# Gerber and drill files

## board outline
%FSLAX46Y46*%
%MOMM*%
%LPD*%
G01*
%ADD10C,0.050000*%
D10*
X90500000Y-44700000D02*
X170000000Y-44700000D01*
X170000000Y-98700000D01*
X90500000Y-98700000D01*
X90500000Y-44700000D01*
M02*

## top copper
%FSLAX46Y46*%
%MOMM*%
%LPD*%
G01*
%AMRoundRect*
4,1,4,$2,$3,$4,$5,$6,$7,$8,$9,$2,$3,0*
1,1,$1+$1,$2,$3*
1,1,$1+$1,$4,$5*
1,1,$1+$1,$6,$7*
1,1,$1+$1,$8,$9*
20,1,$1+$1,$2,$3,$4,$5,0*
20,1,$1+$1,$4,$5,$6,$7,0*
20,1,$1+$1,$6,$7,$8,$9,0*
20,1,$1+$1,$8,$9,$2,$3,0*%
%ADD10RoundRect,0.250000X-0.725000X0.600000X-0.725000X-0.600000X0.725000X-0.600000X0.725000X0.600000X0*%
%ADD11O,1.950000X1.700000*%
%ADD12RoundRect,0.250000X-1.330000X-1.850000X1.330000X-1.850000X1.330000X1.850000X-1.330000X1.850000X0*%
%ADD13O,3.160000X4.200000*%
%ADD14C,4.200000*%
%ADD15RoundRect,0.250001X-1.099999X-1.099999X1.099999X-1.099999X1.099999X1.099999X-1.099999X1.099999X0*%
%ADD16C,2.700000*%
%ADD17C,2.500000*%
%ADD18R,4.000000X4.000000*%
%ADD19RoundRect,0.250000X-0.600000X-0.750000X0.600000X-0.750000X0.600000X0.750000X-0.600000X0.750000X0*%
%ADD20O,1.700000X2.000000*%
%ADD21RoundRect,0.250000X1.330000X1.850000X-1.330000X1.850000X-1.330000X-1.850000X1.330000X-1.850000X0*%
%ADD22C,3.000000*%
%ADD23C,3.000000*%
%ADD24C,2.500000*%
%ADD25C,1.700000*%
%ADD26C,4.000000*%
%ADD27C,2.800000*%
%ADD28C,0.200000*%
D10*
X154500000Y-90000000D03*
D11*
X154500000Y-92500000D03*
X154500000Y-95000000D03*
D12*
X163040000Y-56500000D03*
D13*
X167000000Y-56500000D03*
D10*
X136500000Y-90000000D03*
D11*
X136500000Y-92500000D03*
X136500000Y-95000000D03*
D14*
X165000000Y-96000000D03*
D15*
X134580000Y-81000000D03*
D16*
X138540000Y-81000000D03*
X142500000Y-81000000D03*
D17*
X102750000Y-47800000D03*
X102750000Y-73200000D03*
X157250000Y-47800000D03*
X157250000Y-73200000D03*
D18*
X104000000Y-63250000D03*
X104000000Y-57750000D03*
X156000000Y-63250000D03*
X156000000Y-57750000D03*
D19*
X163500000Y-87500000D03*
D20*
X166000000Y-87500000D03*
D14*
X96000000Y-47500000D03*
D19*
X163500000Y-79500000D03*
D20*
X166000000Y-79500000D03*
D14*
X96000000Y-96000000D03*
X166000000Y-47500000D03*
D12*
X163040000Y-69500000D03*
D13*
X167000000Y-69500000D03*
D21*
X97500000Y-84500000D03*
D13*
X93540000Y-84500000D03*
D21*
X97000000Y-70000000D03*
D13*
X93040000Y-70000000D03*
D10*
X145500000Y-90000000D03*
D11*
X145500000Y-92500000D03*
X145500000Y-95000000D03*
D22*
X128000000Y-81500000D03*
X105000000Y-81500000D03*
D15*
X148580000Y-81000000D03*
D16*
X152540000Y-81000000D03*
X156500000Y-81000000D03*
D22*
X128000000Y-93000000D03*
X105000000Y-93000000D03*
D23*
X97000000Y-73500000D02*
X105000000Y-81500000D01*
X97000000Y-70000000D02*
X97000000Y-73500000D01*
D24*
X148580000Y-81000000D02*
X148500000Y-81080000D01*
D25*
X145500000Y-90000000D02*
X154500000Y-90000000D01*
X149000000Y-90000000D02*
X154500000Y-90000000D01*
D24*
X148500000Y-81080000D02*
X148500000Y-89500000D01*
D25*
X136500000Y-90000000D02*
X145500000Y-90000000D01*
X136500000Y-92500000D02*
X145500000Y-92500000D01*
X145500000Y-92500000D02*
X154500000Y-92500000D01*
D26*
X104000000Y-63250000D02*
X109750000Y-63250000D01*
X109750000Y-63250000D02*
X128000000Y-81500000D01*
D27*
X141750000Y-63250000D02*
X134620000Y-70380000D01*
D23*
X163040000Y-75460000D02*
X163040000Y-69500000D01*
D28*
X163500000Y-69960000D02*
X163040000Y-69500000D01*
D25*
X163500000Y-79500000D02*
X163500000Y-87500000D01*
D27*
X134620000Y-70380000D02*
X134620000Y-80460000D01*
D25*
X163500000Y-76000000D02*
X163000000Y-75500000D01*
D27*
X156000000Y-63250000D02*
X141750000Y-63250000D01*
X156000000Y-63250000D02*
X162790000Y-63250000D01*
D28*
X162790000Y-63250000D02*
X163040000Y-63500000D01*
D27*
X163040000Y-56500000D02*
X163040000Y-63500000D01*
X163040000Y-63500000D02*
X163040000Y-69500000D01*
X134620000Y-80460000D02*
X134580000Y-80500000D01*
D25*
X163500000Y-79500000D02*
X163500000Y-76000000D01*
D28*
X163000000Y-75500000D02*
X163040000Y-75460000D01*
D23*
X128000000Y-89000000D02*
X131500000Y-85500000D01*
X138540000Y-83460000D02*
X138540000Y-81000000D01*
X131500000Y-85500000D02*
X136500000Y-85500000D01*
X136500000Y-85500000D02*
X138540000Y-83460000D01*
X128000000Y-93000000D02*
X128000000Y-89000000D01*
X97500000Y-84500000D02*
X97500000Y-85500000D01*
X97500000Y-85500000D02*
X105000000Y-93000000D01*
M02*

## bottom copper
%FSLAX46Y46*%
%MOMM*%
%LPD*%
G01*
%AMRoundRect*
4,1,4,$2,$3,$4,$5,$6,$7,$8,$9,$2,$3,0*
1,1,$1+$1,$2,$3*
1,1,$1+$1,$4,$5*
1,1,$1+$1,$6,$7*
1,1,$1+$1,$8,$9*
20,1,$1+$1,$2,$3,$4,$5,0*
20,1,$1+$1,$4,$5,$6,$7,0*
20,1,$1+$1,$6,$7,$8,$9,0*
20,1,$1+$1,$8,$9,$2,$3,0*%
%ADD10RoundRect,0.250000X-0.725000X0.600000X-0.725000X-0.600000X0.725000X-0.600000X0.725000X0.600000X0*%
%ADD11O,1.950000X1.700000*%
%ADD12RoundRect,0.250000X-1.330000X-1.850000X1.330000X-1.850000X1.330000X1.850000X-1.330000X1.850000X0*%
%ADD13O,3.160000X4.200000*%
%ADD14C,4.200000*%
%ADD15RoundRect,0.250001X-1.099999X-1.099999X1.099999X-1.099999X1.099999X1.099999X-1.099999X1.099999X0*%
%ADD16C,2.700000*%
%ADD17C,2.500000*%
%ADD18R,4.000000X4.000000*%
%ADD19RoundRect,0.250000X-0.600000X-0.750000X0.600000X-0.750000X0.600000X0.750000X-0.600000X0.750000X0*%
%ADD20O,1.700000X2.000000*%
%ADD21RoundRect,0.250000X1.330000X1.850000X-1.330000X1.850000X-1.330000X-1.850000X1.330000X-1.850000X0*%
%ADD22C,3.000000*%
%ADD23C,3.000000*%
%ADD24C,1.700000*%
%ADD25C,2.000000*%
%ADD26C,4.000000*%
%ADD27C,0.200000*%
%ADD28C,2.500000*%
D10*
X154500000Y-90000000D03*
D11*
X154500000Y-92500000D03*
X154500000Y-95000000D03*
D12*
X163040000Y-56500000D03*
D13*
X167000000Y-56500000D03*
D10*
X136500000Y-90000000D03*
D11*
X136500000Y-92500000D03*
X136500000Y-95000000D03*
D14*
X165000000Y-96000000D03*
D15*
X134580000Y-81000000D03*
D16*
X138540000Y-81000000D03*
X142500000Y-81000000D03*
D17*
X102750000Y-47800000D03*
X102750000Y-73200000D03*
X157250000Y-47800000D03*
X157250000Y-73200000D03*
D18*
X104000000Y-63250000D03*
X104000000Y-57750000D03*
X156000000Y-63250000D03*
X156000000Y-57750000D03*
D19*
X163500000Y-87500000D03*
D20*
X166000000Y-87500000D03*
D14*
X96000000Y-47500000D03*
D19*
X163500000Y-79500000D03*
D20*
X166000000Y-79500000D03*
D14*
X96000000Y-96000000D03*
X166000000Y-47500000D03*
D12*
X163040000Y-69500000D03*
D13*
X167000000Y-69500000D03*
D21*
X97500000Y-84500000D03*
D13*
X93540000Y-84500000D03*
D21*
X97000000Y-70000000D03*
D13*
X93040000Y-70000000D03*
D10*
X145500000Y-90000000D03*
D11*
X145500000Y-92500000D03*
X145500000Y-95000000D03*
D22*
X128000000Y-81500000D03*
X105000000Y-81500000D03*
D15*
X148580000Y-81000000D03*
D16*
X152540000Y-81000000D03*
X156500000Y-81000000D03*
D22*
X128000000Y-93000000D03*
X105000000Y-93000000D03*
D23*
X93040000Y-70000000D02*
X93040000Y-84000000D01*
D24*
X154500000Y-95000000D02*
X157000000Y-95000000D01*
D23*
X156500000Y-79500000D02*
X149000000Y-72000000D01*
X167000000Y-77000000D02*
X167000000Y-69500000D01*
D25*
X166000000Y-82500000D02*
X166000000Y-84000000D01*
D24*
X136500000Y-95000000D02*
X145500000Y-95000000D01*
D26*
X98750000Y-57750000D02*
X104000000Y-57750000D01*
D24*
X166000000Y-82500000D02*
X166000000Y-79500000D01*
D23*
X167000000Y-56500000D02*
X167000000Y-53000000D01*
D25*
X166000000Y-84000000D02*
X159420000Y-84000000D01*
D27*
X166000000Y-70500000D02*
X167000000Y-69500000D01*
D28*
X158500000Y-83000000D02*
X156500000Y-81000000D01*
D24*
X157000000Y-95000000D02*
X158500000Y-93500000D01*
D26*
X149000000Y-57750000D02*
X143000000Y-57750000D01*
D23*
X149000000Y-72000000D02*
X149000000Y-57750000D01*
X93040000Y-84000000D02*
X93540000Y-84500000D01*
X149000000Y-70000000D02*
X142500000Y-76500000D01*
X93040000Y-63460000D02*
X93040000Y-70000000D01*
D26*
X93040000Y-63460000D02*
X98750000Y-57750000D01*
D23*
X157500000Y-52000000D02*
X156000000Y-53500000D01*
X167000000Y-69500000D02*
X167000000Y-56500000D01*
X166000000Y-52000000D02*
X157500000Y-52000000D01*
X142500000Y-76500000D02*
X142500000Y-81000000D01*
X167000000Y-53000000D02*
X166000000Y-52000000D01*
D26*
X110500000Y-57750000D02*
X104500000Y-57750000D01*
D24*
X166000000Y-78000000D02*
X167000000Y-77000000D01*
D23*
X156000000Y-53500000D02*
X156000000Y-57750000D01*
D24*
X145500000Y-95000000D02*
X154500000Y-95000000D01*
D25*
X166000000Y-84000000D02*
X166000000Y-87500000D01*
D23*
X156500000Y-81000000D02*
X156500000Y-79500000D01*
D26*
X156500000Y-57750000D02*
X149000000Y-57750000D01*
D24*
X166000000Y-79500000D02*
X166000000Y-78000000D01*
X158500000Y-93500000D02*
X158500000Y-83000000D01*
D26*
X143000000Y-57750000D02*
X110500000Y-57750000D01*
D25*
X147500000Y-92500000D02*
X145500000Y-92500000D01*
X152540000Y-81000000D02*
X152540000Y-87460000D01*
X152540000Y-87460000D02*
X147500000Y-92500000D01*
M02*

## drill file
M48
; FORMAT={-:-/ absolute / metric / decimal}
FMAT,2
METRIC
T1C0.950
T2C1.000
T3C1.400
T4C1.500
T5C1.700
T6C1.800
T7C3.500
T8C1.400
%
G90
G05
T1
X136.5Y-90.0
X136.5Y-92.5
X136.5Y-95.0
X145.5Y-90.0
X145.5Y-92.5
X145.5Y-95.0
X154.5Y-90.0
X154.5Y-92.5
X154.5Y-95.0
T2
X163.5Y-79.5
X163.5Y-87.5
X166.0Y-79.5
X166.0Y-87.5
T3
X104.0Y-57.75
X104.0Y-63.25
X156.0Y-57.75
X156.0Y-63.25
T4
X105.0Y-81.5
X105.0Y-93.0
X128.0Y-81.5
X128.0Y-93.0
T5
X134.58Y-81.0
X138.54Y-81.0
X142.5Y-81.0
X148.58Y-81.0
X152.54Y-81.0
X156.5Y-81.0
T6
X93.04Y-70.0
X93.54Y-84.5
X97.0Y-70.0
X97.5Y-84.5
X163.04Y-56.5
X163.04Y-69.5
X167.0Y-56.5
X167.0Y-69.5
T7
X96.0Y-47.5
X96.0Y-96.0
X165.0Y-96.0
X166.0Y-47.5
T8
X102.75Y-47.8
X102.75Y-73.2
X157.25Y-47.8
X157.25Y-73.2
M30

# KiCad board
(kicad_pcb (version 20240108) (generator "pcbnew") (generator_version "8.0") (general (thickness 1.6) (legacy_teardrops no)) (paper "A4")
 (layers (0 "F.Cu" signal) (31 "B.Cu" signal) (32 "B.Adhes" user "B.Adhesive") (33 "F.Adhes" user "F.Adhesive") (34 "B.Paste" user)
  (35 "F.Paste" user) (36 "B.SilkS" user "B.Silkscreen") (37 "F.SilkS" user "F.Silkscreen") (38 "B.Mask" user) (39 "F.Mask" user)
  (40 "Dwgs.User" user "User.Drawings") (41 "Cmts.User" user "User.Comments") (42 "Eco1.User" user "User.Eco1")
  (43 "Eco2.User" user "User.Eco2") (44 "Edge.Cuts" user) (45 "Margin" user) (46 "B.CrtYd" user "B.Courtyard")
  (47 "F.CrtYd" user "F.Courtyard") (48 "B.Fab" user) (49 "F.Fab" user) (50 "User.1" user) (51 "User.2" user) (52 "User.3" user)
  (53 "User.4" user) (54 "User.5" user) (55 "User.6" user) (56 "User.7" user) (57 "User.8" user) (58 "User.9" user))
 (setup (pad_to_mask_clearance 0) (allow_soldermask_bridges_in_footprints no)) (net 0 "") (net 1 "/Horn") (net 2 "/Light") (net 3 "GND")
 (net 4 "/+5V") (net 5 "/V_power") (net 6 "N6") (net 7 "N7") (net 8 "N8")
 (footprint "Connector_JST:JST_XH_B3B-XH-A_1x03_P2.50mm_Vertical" (layer "F.Cu") (at 154.5 90 -90)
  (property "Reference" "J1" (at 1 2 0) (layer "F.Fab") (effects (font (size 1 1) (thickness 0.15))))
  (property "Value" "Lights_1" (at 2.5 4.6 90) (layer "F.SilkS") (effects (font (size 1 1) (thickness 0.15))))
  (pad "1" thru_hole roundrect (at 0 0 270) (size 1.7 1.95) (drill 0.95) (layers "*.Cu" "*.Mask") (remove_unused_layers no)
   (roundrect_rratio 0.147059) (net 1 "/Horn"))
  (pad "2" thru_hole oval (at 2.5 0 270) (size 1.7 1.95) (drill 0.95) (layers "*.Cu" "*.Mask") (remove_unused_layers no) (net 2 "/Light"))
  (pad "3" thru_hole oval (at 5 0 270) (size 1.7 1.95) (drill 0.95) (layers "*.Cu" "*.Mask") (remove_unused_layers no) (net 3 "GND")))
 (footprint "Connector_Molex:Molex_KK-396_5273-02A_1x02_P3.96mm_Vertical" (layer "F.Cu") (at 163.04 56.5)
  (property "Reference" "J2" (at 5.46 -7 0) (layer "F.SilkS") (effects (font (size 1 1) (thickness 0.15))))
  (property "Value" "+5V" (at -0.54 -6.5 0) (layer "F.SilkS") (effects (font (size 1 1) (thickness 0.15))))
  (pad "1" thru_hole roundrect (at 0 0) (size 3.16 4.2) (drill 1.8) (layers "*.Cu" "*.Mask") (remove_unused_layers no)
   (roundrect_rratio 0.079114) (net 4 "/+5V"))
  (pad "2" thru_hole oval (at 3.96 0) (size 3.16 4.2) (drill 1.8) (layers "*.Cu" "*.Mask") (remove_unused_layers no) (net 3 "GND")))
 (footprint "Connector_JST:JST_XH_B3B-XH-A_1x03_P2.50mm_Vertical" (layer "F.Cu") (at 136.5 90 -90)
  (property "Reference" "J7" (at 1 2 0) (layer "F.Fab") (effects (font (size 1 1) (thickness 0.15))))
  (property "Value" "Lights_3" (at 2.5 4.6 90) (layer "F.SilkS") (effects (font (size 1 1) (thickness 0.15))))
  (pad "1" thru_hole roundrect (at 0 0 270) (size 1.7 1.95) (drill 0.95) (layers "*.Cu" "*.Mask") (remove_unused_layers no)
   (roundrect_rratio 0.147059) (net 1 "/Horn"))
  (pad "2" thru_hole oval (at 2.5 0 270) (size 1.7 1.95) (drill 0.95) (layers "*.Cu" "*.Mask") (remove_unused_layers no) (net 2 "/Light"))
  (pad "3" thru_hole oval (at 5 0 270) (size 1.7 1.95) (drill 0.95) (layers "*.Cu" "*.Mask") (remove_unused_layers no) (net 3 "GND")))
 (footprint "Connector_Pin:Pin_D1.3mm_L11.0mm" (layer "F.Cu") (at 165 96)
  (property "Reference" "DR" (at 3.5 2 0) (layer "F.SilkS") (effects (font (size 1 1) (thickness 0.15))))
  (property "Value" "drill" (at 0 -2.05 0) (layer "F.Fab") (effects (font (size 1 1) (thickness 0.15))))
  (pad "1" thru_hole circle (at 0 0) (size 4.2 4.2) (drill 3.5) (layers "*.Cu" "*.Mask") (remove_unused_layers no)))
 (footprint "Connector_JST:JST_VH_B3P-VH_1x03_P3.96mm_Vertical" (layer "F.Cu") (at 134.58 81)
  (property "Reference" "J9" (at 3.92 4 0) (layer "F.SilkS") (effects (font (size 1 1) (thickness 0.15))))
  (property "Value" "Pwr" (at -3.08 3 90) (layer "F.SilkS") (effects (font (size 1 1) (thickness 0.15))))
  (pad "1" thru_hole roundrect (at 0 0) (size 2.7 2.7) (drill 1.7) (layers "*.Cu" "*.Mask") (remove_unused_layers no)
   (roundrect_rratio 0.092593) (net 4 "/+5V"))
  (pad "2" thru_hole circle (at 3.96 0) (size 2.7 2.7) (drill 1.7) (layers "*.Cu" "*.Mask") (remove_unused_layers no) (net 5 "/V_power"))
  (pad "3" thru_hole circle (at 7.92 0) (size 2.7 2.7) (drill 1.7) (layers "*.Cu" "*.Mask") (remove_unused_layers no) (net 3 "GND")))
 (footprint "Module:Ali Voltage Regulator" (layer "F.Cu") (at 100 45.5)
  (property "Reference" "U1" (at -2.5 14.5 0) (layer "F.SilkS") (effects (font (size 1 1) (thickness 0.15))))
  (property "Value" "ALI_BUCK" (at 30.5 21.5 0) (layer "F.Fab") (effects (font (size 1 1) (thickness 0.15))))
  (pad "" np_thru_hole circle (at 2.75 2.3) (size 2.5 2.5) (drill 1.4) (layers "*.Cu" "*.Mask") (thermal_bridge_angle 90))
  (pad "" np_thru_hole circle (at 2.75 27.7) (size 2.5 2.5) (drill 1.4) (layers "*.Cu" "*.Mask"))
  (pad "" np_thru_hole circle (at 57.25 2.3) (size 2.5 2.5) (drill 1.4) (layers "*.Cu" "*.Mask"))
  (pad "" np_thru_hole circle (at 57.25 27.7) (size 2.5 2.5) (drill 1.4) (layers "*.Cu" "*.Mask"))
  (pad "1" thru_hole rect (at 4 17.75) (size 4 4) (drill 1.4) (layers "*.Cu" "*.Mask") (remove_unused_layers no) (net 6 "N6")
   (thermal_bridge_angle 45))
  (pad "2" thru_hole rect (at 4 12.25) (size 4 4) (drill 1.4) (layers "*.Cu" "*.Mask") (remove_unused_layers no) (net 3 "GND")
   (thermal_bridge_angle 45))
  (pad "3" thru_hole rect (at 56 17.75) (size 4 4) (drill 1.4) (layers "*.Cu" "*.Mask") (remove_unused_layers no) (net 4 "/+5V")
   (thermal_bridge_angle 45))
  (pad "4" thru_hole rect (at 56 12.25) (size 4 4) (drill 1.4) (layers "*.Cu" "*.Mask") (remove_unused_layers no) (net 3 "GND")
   (thermal_bridge_angle 45)))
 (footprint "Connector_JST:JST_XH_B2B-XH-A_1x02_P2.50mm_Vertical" (layer "F.Cu") (at 163.5 87.5)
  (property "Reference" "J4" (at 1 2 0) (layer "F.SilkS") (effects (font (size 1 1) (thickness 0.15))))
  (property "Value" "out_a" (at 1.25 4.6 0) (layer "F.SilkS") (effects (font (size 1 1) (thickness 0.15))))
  (pad "1" thru_hole roundrect (at 0 0) (size 1.7 2) (drill 1) (layers "*.Cu" "*.Mask") (remove_unused_layers no)
   (roundrect_rratio 0.147059) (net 4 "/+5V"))
  (pad "2" thru_hole oval (at 2.5 0) (size 1.7 2) (drill 1) (layers "*.Cu" "*.Mask") (remove_unused_layers no) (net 3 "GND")))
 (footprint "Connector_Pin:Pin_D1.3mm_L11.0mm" (layer "F.Cu") (at 96 47.5)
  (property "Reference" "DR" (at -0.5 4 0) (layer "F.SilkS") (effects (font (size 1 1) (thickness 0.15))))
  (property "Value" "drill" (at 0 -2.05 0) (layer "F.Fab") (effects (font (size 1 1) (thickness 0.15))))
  (pad "1" thru_hole circle (at 0 0) (size 4.2 4.2) (drill 3.5) (layers "*.Cu" "*.Mask") (remove_unused_layers no)))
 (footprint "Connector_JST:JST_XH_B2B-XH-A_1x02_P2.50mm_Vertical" (layer "F.Cu") (at 163.5 79.5)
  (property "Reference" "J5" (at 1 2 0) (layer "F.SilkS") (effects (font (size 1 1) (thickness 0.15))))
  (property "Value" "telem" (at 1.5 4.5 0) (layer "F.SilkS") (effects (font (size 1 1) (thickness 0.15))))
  (pad "1" thru_hole roundrect (at 0 0) (size 1.7 2) (drill 1) (layers "*.Cu" "*.Mask") (remove_unused_layers no)
   (roundrect_rratio 0.147059) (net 4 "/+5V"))
  (pad "2" thru_hole oval (at 2.5 0) (size 1.7 2) (drill 1) (layers "*.Cu" "*.Mask") (remove_unused_layers no) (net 3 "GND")))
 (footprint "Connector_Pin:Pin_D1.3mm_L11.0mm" (layer "F.Cu") (at 96 96)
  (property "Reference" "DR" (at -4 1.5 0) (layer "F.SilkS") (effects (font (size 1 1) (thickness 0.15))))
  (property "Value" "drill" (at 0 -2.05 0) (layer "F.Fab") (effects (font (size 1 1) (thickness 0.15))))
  (pad "1" thru_hole circle (at 0 0) (size 4.2 4.2) (drill 3.5) (layers "*.Cu" "*.Mask") (remove_unused_layers no)))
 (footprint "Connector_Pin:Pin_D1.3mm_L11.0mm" (layer "F.Cu") (at 166 47.5)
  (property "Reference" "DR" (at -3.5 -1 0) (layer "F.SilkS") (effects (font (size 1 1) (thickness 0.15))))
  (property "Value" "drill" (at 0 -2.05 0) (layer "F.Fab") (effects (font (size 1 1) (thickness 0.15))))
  (pad "1" thru_hole circle (at 0 0) (size 4.2 4.2) (drill 3.5) (layers "*.Cu" "*.Mask") (remove_unused_layers no)))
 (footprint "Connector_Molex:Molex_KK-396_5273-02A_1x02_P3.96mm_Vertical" (layer "F.Cu") (at 163.04 69.5)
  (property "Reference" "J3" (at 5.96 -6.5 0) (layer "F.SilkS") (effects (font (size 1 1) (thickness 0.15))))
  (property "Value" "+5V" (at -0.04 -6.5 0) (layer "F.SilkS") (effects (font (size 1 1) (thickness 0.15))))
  (pad "1" thru_hole roundrect (at 0 0) (size 3.16 4.2) (drill 1.8) (layers "*.Cu" "*.Mask") (remove_unused_layers no)
   (roundrect_rratio 0.079114) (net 4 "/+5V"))
  (pad "2" thru_hole oval (at 3.96 0) (size 3.16 4.2) (drill 1.8) (layers "*.Cu" "*.Mask") (remove_unused_layers no) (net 3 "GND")))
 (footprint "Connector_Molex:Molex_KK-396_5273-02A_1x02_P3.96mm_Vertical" (layer "F.Cu") (at 97.5 84.5 180)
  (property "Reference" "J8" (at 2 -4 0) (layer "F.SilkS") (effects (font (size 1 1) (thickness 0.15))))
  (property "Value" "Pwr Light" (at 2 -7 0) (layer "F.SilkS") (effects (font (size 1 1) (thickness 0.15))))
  (pad "1" thru_hole roundrect (at 0 0 180) (size 3.16 4.2) (drill 1.8) (layers "*.Cu" "*.Mask") (remove_unused_layers no)
   (roundrect_rratio 0.079114) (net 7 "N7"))
  (pad "2" thru_hole oval (at 3.96 0 180) (size 3.16 4.2) (drill 1.8) (layers "*.Cu" "*.Mask") (remove_unused_layers no) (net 3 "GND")))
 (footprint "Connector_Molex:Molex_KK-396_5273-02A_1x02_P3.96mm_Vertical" (layer "F.Cu") (at 97 70 180)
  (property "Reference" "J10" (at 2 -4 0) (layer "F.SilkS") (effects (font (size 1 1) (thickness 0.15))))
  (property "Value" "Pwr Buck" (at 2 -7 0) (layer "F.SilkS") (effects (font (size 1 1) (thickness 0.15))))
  (pad "1" thru_hole roundrect (at 0 0 180) (size 3.16 4.2) (drill 1.8) (layers "*.Cu" "*.Mask") (remove_unused_layers no)
   (roundrect_rratio 0.079114) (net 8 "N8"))
  (pad "2" thru_hole oval (at 3.96 0 180) (size 3.16 4.2) (drill 1.8) (layers "*.Cu" "*.Mask") (remove_unused_layers no) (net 3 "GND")))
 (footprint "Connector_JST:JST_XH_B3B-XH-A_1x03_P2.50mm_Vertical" (layer "F.Cu") (at 145.5 90 -90)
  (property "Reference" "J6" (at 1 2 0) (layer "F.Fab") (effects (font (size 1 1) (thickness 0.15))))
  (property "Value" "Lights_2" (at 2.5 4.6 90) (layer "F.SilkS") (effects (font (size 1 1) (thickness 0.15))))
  (pad "1" thru_hole roundrect (at 0 0 270) (size 1.7 1.95) (drill 0.95) (layers "*.Cu" "*.Mask") (remove_unused_layers no)
   (roundrect_rratio 0.147059) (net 1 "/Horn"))
  (pad "2" thru_hole oval (at 2.5 0 270) (size 1.7 1.95) (drill 0.95) (layers "*.Cu" "*.Mask") (remove_unused_layers no) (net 2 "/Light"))
  (pad "3" thru_hole oval (at 5 0 270) (size 1.7 1.95) (drill 0.95) (layers "*.Cu" "*.Mask") (remove_unused_layers no) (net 3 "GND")))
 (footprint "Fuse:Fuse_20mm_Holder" (layer "F.Cu") (at 128 81.5 180)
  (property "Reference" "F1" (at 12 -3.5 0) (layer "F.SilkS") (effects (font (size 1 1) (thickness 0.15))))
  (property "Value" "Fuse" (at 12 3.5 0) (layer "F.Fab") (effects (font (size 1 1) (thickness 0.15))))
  (pad "1" thru_hole circle (at 0 0 180) (size 3 3) (drill 1.5) (layers "*.Cu" "*.Mask") (remove_unused_layers no) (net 6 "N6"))
  (pad "2" thru_hole circle (at 23 0 180) (size 3 3) (drill 1.5) (layers "*.Cu" "*.Mask") (remove_unused_layers no) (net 8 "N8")))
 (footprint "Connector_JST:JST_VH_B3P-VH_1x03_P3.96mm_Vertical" (layer "F.Cu") (at 148.58 81)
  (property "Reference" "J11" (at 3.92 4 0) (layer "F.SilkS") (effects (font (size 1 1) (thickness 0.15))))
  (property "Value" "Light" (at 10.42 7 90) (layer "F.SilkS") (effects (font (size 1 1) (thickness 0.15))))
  (pad "1" thru_hole roundrect (at 0 0) (size 2.7 2.7) (drill 1.7) (layers "*.Cu" "*.Mask") (remove_unused_layers no)
   (roundrect_rratio 0.092593) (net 1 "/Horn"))
  (pad "2" thru_hole circle (at 3.96 0) (size 2.7 2.7) (drill 1.7) (layers "*.Cu" "*.Mask") (remove_unused_layers no) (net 2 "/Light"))
  (pad "3" thru_hole circle (at 7.92 0) (size 2.7 2.7) (drill 1.7) (layers "*.Cu" "*.Mask") (remove_unused_layers no) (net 3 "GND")))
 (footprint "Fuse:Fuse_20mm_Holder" (layer "F.Cu") (at 128 93 180)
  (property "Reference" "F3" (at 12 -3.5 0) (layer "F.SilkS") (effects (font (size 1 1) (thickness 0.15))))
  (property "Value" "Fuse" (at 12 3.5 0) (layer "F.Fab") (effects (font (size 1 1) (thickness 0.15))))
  (pad "1" thru_hole circle (at 0 0 180) (size 3 3) (drill 1.5) (layers "*.Cu" "*.Mask") (remove_unused_layers no) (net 5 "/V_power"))
  (pad "2" thru_hole circle (at 23 0 180) (size 3 3) (drill 1.5) (layers "*.Cu" "*.Mask") (remove_unused_layers no) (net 7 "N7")))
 (gr_rect (start 90.5 44.7) (end 170 98.7) (stroke (width 0.05) (type default)) (fill none) (layer "Edge.Cuts"))
 (segment (start 93.04 70) (end 93.04 84) (width 3) (layer "B.Cu") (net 3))
 (segment (start 154.5 95) (end 157 95) (width 1.7) (layer "B.Cu") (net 3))
 (segment (start 156.5 79.5) (end 149 72) (width 3) (layer "B.Cu") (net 3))
 (segment (start 167 77) (end 167 69.5) (width 3) (layer "B.Cu") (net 3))
 (segment (start 166 82.5) (end 166 84) (width 2) (layer "B.Cu") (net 3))
 (segment (start 136.5 95) (end 145.5 95) (width 1.7) (layer "B.Cu") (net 3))
 (segment (start 98.75 57.75) (end 104 57.75) (width 4) (layer "B.Cu") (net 3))
 (segment (start 166 82.5) (end 166 79.5) (width 1.7) (layer "B.Cu") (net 3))
 (segment (start 167 56.5) (end 167 53) (width 3) (layer "B.Cu") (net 3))
 (segment (start 166 84) (end 159.42 84) (width 2) (layer "B.Cu") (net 3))
 (segment (start 166 70.5) (end 167 69.5) (width 0.2) (layer "B.Cu") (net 3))
 (segment (start 158.5 83) (end 156.5 81) (width 2.5) (layer "B.Cu") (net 3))
 (segment (start 157 95) (end 158.5 93.5) (width 1.7) (layer "B.Cu") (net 3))
 (segment (start 149 57.75) (end 143 57.75) (width 4) (layer "B.Cu") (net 3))
 (segment (start 149 72) (end 149 57.75) (width 3) (layer "B.Cu") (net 3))
 (segment (start 93.04 84) (end 93.54 84.5) (width 3) (layer "B.Cu") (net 3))
 (segment (start 149 70) (end 142.5 76.5) (width 3) (layer "B.Cu") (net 3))
 (segment (start 93.04 63.46) (end 93.04 70) (width 3) (layer "B.Cu") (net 3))
 (segment (start 93.04 63.46) (end 98.75 57.75) (width 4) (layer "B.Cu") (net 3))
 (segment (start 157.5 52) (end 156 53.5) (width 3) (layer "B.Cu") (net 3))
 (segment (start 167 69.5) (end 167 56.5) (width 3) (layer "B.Cu") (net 3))
 (segment (start 166 52) (end 157.5 52) (width 3) (layer "B.Cu") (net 3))
 (segment (start 142.5 76.5) (end 142.5 81) (width 3) (layer "B.Cu") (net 3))
 (segment (start 167 53) (end 166 52) (width 3) (layer "B.Cu") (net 3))
 (segment (start 110.5 57.75) (end 104.5 57.75) (width 4) (layer "B.Cu") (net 3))
 (segment (start 166 78) (end 167 77) (width 1.7) (layer "B.Cu") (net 3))
 (segment (start 156 53.5) (end 156 57.75) (width 3) (layer "B.Cu") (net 3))
 (segment (start 145.5 95) (end 154.5 95) (width 1.7) (layer "B.Cu") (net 3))
 (segment (start 166 84) (end 166 87.5) (width 2) (layer "B.Cu") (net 3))
 (segment (start 156.5 81) (end 156.5 79.5) (width 3) (layer "B.Cu") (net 3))
 (segment (start 156.5 57.75) (end 149 57.75) (width 4) (layer "B.Cu") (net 3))
 (segment (start 166 79.5) (end 166 78) (width 1.7) (layer "B.Cu") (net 3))
 (segment (start 158.5 93.5) (end 158.5 83) (width 1.7) (layer "B.Cu") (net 3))
 (segment (start 143 57.75) (end 110.5 57.75) (width 4) (layer "B.Cu") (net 3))
 (segment (start 97 73.5) (end 105 81.5) (width 3) (layer "F.Cu") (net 8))
 (segment (start 97 70) (end 97 73.5) (width 3) (layer "F.Cu") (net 8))
 (segment (start 148.58 81) (end 148.5 81.08) (width 2.5) (layer "F.Cu") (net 1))
 (segment (start 145.5 90) (end 154.5 90) (width 1.7) (layer "F.Cu") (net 1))
 (segment (start 149 90) (end 154.5 90) (width 1.7) (layer "F.Cu") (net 1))
 (segment (start 148.5 81.08) (end 148.5 89.5) (width 2.5) (layer "F.Cu") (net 1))
 (segment (start 136.5 90) (end 145.5 90) (width 1.7) (layer "F.Cu") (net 1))
 (segment (start 136.5 92.5) (end 145.5 92.5) (width 1.7) (layer "F.Cu") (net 2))
 (segment (start 145.5 92.5) (end 154.5 92.5) (width 1.7) (layer "F.Cu") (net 2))
 (segment (start 147.5 92.5) (end 145.5 92.5) (width 2) (layer "B.Cu") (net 2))
 (segment (start 152.54 81) (end 152.54 87.46) (width 2) (layer "B.Cu") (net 2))
 (segment (start 152.54 87.46) (end 147.5 92.5) (width 2) (layer "B.Cu") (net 2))
 (segment (start 104 63.25) (end 109.75 63.25) (width 4) (layer "F.Cu") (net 6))
 (segment (start 109.75 63.25) (end 128 81.5) (width 4) (layer "F.Cu") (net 6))
 (segment (start 141.75 63.25) (end 134.62 70.38) (width 2.8) (layer "F.Cu") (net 4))
 (segment (start 163.04 75.46) (end 163.04 69.5) (width 3) (layer "F.Cu") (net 4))
 (segment (start 163.5 69.96) (end 163.04 69.5) (width 0.2) (layer "F.Cu") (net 4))
 (segment (start 163.5 79.5) (end 163.5 87.5) (width 1.7) (layer "F.Cu") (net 4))
 (segment (start 134.62 70.38) (end 134.62 80.46) (width 2.8) (layer "F.Cu") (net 4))
 (segment (start 163.5 76) (end 163 75.5) (width 1.7) (layer "F.Cu") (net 4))
 (segment (start 156 63.25) (end 141.75 63.25) (width 2.8) (layer "F.Cu") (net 4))
 (segment (start 156 63.25) (end 162.79 63.25) (width 2.8) (layer "F.Cu") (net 4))
 (segment (start 162.79 63.25) (end 163.04 63.5) (width 0.2) (layer "F.Cu") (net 4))
 (segment (start 163.04 56.5) (end 163.04 63.5) (width 2.8) (layer "F.Cu") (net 4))
 (segment (start 163.04 63.5) (end 163.04 69.5) (width 2.8) (layer "F.Cu") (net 4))
 (segment (start 134.62 80.46) (end 134.58 80.5) (width 2.8) (layer "F.Cu") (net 4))
 (segment (start 163.5 79.5) (end 163.5 76) (width 1.7) (layer "F.Cu") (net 4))
 (segment (start 163 75.5) (end 163.04 75.46) (width 0.2) (layer "F.Cu") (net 4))
 (segment (start 128 89) (end 131.5 85.5) (width 3) (layer "F.Cu") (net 5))
 (segment (start 138.54 83.46) (end 138.54 81) (width 3) (layer "F.Cu") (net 5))
 (segment (start 131.5 85.5) (end 136.5 85.5) (width 3) (layer "F.Cu") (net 5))
 (segment (start 136.5 85.5) (end 138.54 83.46) (width 3) (layer "F.Cu") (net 5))
 (segment (start 128 93) (end 128 89) (width 3) (layer "F.Cu") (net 5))
 (segment (start 97.5 84.5) (end 97.5 85.5) (width 3) (layer "F.Cu") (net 7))
 (segment (start 97.5 85.5) (end 105 93) (width 3) (layer "F.Cu") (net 7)))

